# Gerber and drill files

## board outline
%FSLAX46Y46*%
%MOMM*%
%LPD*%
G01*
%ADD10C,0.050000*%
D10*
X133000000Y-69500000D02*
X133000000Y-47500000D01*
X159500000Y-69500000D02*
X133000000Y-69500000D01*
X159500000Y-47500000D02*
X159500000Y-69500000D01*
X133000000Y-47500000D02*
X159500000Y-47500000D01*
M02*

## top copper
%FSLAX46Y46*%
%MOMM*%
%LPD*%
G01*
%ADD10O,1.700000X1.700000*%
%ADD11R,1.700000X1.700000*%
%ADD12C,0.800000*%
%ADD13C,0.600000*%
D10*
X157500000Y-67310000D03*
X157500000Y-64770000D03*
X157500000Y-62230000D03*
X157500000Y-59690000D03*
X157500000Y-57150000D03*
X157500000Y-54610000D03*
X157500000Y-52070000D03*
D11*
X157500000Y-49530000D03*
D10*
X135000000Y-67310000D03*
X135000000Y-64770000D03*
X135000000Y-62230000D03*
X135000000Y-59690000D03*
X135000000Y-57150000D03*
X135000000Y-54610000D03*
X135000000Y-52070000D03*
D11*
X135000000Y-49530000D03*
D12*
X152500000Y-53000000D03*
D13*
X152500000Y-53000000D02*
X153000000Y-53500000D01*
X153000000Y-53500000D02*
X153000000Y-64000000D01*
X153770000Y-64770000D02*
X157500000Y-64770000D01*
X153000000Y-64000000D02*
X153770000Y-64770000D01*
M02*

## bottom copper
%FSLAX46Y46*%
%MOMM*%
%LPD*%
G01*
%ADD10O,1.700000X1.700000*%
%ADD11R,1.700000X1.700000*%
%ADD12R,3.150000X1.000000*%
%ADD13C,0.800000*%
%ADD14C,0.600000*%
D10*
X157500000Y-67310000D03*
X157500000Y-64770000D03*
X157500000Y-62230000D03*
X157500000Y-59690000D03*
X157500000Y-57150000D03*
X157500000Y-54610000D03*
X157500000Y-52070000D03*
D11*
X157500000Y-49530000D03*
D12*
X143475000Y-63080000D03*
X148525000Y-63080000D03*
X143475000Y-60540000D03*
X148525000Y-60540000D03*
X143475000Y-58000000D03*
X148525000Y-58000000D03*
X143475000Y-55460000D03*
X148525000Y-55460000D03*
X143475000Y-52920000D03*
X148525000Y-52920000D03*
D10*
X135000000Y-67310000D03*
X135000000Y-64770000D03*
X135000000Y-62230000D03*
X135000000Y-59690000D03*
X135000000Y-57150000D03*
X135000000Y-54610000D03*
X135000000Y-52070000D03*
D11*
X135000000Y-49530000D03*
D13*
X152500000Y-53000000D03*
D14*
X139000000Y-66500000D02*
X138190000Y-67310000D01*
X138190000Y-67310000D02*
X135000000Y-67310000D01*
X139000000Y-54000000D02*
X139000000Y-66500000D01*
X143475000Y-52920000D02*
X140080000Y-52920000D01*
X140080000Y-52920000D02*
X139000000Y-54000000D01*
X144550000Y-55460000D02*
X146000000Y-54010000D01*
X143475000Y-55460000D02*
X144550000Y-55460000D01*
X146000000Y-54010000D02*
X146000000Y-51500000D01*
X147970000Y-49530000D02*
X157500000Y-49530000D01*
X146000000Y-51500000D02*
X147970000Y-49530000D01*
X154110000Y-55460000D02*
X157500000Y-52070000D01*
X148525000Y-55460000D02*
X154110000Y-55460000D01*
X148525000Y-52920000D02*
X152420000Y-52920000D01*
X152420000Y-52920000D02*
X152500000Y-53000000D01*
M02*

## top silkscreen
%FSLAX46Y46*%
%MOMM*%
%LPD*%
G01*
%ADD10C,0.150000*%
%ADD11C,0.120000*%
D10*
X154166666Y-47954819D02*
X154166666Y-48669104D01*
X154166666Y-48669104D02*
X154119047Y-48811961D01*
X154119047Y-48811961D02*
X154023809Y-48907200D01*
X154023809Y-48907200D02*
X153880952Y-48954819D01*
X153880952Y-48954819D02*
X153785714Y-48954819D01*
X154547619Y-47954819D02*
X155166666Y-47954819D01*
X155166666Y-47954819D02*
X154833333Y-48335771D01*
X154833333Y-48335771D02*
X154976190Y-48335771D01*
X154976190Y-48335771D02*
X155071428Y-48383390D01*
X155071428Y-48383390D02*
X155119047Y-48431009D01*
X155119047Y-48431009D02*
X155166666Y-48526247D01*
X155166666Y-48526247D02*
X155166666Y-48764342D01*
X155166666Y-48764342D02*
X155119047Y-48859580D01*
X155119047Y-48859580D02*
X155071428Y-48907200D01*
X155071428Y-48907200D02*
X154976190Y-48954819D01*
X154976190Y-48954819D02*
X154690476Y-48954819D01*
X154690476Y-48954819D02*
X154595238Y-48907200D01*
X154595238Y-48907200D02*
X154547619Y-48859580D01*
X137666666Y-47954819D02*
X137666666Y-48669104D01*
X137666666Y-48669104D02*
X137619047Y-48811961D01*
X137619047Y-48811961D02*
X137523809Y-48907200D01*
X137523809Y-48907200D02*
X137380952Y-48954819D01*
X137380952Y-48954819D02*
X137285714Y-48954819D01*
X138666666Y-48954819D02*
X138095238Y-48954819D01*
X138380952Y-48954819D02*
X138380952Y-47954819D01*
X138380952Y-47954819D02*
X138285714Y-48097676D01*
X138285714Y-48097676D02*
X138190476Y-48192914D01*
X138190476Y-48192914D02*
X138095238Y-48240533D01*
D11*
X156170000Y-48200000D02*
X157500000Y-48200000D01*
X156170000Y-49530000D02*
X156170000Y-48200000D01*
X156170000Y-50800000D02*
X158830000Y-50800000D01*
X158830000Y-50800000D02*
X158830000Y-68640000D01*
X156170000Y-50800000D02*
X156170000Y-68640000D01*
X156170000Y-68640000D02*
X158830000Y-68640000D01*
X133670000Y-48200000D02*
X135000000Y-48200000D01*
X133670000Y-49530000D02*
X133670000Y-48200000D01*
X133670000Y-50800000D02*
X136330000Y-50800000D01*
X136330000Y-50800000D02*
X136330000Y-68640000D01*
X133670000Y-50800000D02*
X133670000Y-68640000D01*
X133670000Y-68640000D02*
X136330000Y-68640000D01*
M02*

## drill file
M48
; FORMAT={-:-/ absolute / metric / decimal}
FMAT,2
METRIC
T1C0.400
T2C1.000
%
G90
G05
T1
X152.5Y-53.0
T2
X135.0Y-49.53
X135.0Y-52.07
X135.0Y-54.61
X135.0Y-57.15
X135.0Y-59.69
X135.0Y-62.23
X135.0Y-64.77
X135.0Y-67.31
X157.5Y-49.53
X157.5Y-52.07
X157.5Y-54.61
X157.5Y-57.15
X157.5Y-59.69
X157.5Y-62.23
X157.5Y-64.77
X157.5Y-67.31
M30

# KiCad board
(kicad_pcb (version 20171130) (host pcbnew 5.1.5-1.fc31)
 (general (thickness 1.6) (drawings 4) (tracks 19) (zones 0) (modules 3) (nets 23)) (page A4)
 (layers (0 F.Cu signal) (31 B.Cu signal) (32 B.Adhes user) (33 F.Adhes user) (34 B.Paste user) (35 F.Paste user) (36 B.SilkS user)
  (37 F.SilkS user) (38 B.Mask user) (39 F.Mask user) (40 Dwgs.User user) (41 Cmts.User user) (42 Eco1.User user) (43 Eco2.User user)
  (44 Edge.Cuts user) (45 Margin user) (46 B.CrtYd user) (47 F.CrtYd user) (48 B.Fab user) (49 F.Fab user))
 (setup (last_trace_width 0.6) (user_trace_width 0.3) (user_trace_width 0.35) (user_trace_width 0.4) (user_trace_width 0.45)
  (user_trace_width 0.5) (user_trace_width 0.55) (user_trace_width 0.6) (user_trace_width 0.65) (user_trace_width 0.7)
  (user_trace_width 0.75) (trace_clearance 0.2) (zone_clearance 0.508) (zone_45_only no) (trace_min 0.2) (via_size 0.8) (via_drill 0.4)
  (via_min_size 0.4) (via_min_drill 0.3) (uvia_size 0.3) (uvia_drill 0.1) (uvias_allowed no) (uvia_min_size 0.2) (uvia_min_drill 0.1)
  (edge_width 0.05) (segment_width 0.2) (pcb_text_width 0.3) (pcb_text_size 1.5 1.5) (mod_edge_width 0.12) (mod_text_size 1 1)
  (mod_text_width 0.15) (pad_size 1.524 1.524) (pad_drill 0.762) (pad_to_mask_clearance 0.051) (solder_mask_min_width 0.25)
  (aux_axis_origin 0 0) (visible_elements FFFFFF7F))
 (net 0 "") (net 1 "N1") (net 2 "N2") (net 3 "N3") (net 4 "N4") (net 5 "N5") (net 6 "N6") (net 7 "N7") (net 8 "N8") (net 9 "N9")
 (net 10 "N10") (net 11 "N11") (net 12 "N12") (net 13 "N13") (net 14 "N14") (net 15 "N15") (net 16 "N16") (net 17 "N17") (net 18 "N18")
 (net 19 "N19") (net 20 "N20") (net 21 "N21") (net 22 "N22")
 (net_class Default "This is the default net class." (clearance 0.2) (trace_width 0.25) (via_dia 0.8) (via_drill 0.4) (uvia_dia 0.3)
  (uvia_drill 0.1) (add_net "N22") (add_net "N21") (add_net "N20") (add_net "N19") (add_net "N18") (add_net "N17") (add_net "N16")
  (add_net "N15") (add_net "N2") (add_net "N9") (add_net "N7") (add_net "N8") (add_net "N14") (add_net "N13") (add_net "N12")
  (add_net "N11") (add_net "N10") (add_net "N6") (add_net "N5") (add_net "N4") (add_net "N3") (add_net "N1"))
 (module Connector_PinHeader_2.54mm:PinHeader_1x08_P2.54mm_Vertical (layer F.Cu) (at 157.5 49.53)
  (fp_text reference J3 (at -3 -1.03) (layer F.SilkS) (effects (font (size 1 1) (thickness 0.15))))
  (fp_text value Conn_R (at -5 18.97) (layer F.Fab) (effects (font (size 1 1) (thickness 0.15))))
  (fp_line (start -1.33 -1.33) (end 0 -1.33) (layer F.SilkS) (width 0.12))
  (fp_line (start -1.33 0) (end -1.33 -1.33) (layer F.SilkS) (width 0.12))
  (fp_line (start -1.33 1.27) (end 1.33 1.27) (layer F.SilkS) (width 0.12))
  (fp_line (start 1.33 1.27) (end 1.33 19.11) (layer F.SilkS) (width 0.12))
  (fp_line (start -1.33 1.27) (end -1.33 19.11) (layer F.SilkS) (width 0.12))
  (fp_line (start -1.33 19.11) (end 1.33 19.11) (layer F.SilkS) (width 0.12))
  (pad 8 thru_hole oval (at 0 17.78) (size 1.7 1.7) (drill 1) (layers *.Cu *.Mask) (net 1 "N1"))
  (pad 7 thru_hole oval (at 0 15.24) (size 1.7 1.7) (drill 1) (layers *.Cu *.Mask) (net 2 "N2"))
  (pad 6 thru_hole oval (at 0 12.7) (size 1.7 1.7) (drill 1) (layers *.Cu *.Mask) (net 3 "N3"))
  (pad 5 thru_hole oval (at 0 10.16) (size 1.7 1.7) (drill 1) (layers *.Cu *.Mask) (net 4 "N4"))
  (pad 4 thru_hole oval (at 0 7.62) (size 1.7 1.7) (drill 1) (layers *.Cu *.Mask) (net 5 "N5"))
  (pad 3 thru_hole oval (at 0 5.08) (size 1.7 1.7) (drill 1) (layers *.Cu *.Mask) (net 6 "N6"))
  (pad 2 thru_hole oval (at 0 2.54) (size 1.7 1.7) (drill 1) (layers *.Cu *.Mask) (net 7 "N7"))
  (pad 1 thru_hole rect (at 0 0) (size 1.7 1.7) (drill 1) (layers *.Cu *.Mask) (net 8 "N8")))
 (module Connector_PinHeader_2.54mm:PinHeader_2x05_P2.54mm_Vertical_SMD (layer B.Cu) (at 146 58 180)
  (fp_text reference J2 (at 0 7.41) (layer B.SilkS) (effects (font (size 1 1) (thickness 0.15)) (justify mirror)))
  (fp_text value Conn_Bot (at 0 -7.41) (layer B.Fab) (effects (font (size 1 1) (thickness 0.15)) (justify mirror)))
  (pad 10 smd rect (at 2.525 -5.08 180) (size 3.15 1) (layers B.Cu B.Paste B.Mask) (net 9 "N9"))
  (pad 9 smd rect (at -2.525 -5.08 180) (size 3.15 1) (layers B.Cu B.Paste B.Mask) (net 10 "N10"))
  (pad 8 smd rect (at 2.525 -2.54 180) (size 3.15 1) (layers B.Cu B.Paste B.Mask) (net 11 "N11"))
  (pad 7 smd rect (at -2.525 -2.54 180) (size 3.15 1) (layers B.Cu B.Paste B.Mask) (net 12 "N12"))
  (pad 6 smd rect (at 2.525 0 180) (size 3.15 1) (layers B.Cu B.Paste B.Mask) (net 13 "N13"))
  (pad 5 smd rect (at -2.525 0 180) (size 3.15 1) (layers B.Cu B.Paste B.Mask) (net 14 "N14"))
  (pad 4 smd rect (at 2.525 2.54 180) (size 3.15 1) (layers B.Cu B.Paste B.Mask) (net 8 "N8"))
  (pad 3 smd rect (at -2.525 2.54 180) (size 3.15 1) (layers B.Cu B.Paste B.Mask) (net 7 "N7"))
  (pad 2 smd rect (at 2.525 5.08 180) (size 3.15 1) (layers B.Cu B.Paste B.Mask) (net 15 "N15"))
  (pad 1 smd rect (at -2.525 5.08 180) (size 3.15 1) (layers B.Cu B.Paste B.Mask) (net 2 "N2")))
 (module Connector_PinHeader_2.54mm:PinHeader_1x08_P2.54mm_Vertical (layer F.Cu) (at 135 49.53)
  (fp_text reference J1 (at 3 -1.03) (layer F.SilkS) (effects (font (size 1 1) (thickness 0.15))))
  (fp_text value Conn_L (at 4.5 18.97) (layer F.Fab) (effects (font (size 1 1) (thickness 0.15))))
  (fp_line (start -1.33 -1.33) (end 0 -1.33) (layer F.SilkS) (width 0.12))
  (fp_line (start -1.33 0) (end -1.33 -1.33) (layer F.SilkS) (width 0.12))
  (fp_line (start -1.33 1.27) (end 1.33 1.27) (layer F.SilkS) (width 0.12))
  (fp_line (start 1.33 1.27) (end 1.33 19.11) (layer F.SilkS) (width 0.12))
  (fp_line (start -1.33 1.27) (end -1.33 19.11) (layer F.SilkS) (width 0.12))
  (fp_line (start -1.33 19.11) (end 1.33 19.11) (layer F.SilkS) (width 0.12))
  (pad 8 thru_hole oval (at 0 17.78) (size 1.7 1.7) (drill 1) (layers *.Cu *.Mask) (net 15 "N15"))
  (pad 7 thru_hole oval (at 0 15.24) (size 1.7 1.7) (drill 1) (layers *.Cu *.Mask) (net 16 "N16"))
  (pad 6 thru_hole oval (at 0 12.7) (size 1.7 1.7) (drill 1) (layers *.Cu *.Mask) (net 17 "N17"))
  (pad 5 thru_hole oval (at 0 10.16) (size 1.7 1.7) (drill 1) (layers *.Cu *.Mask) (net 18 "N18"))
  (pad 4 thru_hole oval (at 0 7.62) (size 1.7 1.7) (drill 1) (layers *.Cu *.Mask) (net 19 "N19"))
  (pad 3 thru_hole oval (at 0 5.08) (size 1.7 1.7) (drill 1) (layers *.Cu *.Mask) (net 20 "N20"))
  (pad 2 thru_hole oval (at 0 2.54) (size 1.7 1.7) (drill 1) (layers *.Cu *.Mask) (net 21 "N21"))
  (pad 1 thru_hole rect (at 0 0) (size 1.7 1.7) (drill 1) (layers *.Cu *.Mask) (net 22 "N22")))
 (gr_line (start 133 69.5) (end 133 47.5) (layer Edge.Cuts) (width 0.05))
 (gr_line (start 159.5 69.5) (end 133 69.5) (layer Edge.Cuts) (width 0.05))
 (gr_line (start 159.5 47.5) (end 159.5 69.5) (layer Edge.Cuts) (width 0.05))
 (gr_line (start 133 47.5) (end 159.5 47.5) (layer Edge.Cuts) (width 0.05))
 (segment (start 139 66.5) (end 138.19 67.31) (width 0.6) (layer B.Cu) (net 15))
 (segment (start 138.19 67.31) (end 135 67.31) (width 0.6) (layer B.Cu) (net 15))
 (segment (start 139 54) (end 139 66.5) (width 0.6) (layer B.Cu) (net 15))
 (segment (start 143.475 52.92) (end 140.08 52.92) (width 0.6) (layer B.Cu) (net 15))
 (segment (start 140.08 52.92) (end 139 54) (width 0.6) (layer B.Cu) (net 15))
 (segment (start 144.55 55.46) (end 146 54.01) (width 0.6) (layer B.Cu) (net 8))
 (segment (start 143.475 55.46) (end 144.55 55.46) (width 0.6) (layer B.Cu) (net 8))
 (segment (start 146 54.01) (end 146 51.5) (width 0.6) (layer B.Cu) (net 8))
 (segment (start 147.97 49.53) (end 157.5 49.53) (width 0.6) (layer B.Cu) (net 8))
 (segment (start 146 51.5) (end 147.97 49.53) (width 0.6) (layer B.Cu) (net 8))
 (segment (start 154.11 55.46) (end 157.5 52.07) (width 0.6) (layer B.Cu) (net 7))
 (segment (start 148.525 55.46) (end 154.11 55.46) (width 0.6) (layer B.Cu) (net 7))
 (segment (start 148.525 52.92) (end 152.42 52.92) (width 0.6) (layer B.Cu) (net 2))
 (via (at 152.5 53) (size 0.8) (drill 0.4) (layers F.Cu B.Cu) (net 2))
 (segment (start 152.42 52.92) (end 152.5 53) (width 0.6) (layer B.Cu) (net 2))
 (segment (start 152.5 53) (end 153 53.5) (width 0.6) (layer F.Cu) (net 2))
 (segment (start 153 53.5) (end 153 64) (width 0.6) (layer F.Cu) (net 2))
 (segment (start 153.77 64.77) (end 157.5 64.77) (width 0.6) (layer F.Cu) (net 2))
 (segment (start 153 64) (end 153.77 64.77) (width 0.6) (layer F.Cu) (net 2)))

